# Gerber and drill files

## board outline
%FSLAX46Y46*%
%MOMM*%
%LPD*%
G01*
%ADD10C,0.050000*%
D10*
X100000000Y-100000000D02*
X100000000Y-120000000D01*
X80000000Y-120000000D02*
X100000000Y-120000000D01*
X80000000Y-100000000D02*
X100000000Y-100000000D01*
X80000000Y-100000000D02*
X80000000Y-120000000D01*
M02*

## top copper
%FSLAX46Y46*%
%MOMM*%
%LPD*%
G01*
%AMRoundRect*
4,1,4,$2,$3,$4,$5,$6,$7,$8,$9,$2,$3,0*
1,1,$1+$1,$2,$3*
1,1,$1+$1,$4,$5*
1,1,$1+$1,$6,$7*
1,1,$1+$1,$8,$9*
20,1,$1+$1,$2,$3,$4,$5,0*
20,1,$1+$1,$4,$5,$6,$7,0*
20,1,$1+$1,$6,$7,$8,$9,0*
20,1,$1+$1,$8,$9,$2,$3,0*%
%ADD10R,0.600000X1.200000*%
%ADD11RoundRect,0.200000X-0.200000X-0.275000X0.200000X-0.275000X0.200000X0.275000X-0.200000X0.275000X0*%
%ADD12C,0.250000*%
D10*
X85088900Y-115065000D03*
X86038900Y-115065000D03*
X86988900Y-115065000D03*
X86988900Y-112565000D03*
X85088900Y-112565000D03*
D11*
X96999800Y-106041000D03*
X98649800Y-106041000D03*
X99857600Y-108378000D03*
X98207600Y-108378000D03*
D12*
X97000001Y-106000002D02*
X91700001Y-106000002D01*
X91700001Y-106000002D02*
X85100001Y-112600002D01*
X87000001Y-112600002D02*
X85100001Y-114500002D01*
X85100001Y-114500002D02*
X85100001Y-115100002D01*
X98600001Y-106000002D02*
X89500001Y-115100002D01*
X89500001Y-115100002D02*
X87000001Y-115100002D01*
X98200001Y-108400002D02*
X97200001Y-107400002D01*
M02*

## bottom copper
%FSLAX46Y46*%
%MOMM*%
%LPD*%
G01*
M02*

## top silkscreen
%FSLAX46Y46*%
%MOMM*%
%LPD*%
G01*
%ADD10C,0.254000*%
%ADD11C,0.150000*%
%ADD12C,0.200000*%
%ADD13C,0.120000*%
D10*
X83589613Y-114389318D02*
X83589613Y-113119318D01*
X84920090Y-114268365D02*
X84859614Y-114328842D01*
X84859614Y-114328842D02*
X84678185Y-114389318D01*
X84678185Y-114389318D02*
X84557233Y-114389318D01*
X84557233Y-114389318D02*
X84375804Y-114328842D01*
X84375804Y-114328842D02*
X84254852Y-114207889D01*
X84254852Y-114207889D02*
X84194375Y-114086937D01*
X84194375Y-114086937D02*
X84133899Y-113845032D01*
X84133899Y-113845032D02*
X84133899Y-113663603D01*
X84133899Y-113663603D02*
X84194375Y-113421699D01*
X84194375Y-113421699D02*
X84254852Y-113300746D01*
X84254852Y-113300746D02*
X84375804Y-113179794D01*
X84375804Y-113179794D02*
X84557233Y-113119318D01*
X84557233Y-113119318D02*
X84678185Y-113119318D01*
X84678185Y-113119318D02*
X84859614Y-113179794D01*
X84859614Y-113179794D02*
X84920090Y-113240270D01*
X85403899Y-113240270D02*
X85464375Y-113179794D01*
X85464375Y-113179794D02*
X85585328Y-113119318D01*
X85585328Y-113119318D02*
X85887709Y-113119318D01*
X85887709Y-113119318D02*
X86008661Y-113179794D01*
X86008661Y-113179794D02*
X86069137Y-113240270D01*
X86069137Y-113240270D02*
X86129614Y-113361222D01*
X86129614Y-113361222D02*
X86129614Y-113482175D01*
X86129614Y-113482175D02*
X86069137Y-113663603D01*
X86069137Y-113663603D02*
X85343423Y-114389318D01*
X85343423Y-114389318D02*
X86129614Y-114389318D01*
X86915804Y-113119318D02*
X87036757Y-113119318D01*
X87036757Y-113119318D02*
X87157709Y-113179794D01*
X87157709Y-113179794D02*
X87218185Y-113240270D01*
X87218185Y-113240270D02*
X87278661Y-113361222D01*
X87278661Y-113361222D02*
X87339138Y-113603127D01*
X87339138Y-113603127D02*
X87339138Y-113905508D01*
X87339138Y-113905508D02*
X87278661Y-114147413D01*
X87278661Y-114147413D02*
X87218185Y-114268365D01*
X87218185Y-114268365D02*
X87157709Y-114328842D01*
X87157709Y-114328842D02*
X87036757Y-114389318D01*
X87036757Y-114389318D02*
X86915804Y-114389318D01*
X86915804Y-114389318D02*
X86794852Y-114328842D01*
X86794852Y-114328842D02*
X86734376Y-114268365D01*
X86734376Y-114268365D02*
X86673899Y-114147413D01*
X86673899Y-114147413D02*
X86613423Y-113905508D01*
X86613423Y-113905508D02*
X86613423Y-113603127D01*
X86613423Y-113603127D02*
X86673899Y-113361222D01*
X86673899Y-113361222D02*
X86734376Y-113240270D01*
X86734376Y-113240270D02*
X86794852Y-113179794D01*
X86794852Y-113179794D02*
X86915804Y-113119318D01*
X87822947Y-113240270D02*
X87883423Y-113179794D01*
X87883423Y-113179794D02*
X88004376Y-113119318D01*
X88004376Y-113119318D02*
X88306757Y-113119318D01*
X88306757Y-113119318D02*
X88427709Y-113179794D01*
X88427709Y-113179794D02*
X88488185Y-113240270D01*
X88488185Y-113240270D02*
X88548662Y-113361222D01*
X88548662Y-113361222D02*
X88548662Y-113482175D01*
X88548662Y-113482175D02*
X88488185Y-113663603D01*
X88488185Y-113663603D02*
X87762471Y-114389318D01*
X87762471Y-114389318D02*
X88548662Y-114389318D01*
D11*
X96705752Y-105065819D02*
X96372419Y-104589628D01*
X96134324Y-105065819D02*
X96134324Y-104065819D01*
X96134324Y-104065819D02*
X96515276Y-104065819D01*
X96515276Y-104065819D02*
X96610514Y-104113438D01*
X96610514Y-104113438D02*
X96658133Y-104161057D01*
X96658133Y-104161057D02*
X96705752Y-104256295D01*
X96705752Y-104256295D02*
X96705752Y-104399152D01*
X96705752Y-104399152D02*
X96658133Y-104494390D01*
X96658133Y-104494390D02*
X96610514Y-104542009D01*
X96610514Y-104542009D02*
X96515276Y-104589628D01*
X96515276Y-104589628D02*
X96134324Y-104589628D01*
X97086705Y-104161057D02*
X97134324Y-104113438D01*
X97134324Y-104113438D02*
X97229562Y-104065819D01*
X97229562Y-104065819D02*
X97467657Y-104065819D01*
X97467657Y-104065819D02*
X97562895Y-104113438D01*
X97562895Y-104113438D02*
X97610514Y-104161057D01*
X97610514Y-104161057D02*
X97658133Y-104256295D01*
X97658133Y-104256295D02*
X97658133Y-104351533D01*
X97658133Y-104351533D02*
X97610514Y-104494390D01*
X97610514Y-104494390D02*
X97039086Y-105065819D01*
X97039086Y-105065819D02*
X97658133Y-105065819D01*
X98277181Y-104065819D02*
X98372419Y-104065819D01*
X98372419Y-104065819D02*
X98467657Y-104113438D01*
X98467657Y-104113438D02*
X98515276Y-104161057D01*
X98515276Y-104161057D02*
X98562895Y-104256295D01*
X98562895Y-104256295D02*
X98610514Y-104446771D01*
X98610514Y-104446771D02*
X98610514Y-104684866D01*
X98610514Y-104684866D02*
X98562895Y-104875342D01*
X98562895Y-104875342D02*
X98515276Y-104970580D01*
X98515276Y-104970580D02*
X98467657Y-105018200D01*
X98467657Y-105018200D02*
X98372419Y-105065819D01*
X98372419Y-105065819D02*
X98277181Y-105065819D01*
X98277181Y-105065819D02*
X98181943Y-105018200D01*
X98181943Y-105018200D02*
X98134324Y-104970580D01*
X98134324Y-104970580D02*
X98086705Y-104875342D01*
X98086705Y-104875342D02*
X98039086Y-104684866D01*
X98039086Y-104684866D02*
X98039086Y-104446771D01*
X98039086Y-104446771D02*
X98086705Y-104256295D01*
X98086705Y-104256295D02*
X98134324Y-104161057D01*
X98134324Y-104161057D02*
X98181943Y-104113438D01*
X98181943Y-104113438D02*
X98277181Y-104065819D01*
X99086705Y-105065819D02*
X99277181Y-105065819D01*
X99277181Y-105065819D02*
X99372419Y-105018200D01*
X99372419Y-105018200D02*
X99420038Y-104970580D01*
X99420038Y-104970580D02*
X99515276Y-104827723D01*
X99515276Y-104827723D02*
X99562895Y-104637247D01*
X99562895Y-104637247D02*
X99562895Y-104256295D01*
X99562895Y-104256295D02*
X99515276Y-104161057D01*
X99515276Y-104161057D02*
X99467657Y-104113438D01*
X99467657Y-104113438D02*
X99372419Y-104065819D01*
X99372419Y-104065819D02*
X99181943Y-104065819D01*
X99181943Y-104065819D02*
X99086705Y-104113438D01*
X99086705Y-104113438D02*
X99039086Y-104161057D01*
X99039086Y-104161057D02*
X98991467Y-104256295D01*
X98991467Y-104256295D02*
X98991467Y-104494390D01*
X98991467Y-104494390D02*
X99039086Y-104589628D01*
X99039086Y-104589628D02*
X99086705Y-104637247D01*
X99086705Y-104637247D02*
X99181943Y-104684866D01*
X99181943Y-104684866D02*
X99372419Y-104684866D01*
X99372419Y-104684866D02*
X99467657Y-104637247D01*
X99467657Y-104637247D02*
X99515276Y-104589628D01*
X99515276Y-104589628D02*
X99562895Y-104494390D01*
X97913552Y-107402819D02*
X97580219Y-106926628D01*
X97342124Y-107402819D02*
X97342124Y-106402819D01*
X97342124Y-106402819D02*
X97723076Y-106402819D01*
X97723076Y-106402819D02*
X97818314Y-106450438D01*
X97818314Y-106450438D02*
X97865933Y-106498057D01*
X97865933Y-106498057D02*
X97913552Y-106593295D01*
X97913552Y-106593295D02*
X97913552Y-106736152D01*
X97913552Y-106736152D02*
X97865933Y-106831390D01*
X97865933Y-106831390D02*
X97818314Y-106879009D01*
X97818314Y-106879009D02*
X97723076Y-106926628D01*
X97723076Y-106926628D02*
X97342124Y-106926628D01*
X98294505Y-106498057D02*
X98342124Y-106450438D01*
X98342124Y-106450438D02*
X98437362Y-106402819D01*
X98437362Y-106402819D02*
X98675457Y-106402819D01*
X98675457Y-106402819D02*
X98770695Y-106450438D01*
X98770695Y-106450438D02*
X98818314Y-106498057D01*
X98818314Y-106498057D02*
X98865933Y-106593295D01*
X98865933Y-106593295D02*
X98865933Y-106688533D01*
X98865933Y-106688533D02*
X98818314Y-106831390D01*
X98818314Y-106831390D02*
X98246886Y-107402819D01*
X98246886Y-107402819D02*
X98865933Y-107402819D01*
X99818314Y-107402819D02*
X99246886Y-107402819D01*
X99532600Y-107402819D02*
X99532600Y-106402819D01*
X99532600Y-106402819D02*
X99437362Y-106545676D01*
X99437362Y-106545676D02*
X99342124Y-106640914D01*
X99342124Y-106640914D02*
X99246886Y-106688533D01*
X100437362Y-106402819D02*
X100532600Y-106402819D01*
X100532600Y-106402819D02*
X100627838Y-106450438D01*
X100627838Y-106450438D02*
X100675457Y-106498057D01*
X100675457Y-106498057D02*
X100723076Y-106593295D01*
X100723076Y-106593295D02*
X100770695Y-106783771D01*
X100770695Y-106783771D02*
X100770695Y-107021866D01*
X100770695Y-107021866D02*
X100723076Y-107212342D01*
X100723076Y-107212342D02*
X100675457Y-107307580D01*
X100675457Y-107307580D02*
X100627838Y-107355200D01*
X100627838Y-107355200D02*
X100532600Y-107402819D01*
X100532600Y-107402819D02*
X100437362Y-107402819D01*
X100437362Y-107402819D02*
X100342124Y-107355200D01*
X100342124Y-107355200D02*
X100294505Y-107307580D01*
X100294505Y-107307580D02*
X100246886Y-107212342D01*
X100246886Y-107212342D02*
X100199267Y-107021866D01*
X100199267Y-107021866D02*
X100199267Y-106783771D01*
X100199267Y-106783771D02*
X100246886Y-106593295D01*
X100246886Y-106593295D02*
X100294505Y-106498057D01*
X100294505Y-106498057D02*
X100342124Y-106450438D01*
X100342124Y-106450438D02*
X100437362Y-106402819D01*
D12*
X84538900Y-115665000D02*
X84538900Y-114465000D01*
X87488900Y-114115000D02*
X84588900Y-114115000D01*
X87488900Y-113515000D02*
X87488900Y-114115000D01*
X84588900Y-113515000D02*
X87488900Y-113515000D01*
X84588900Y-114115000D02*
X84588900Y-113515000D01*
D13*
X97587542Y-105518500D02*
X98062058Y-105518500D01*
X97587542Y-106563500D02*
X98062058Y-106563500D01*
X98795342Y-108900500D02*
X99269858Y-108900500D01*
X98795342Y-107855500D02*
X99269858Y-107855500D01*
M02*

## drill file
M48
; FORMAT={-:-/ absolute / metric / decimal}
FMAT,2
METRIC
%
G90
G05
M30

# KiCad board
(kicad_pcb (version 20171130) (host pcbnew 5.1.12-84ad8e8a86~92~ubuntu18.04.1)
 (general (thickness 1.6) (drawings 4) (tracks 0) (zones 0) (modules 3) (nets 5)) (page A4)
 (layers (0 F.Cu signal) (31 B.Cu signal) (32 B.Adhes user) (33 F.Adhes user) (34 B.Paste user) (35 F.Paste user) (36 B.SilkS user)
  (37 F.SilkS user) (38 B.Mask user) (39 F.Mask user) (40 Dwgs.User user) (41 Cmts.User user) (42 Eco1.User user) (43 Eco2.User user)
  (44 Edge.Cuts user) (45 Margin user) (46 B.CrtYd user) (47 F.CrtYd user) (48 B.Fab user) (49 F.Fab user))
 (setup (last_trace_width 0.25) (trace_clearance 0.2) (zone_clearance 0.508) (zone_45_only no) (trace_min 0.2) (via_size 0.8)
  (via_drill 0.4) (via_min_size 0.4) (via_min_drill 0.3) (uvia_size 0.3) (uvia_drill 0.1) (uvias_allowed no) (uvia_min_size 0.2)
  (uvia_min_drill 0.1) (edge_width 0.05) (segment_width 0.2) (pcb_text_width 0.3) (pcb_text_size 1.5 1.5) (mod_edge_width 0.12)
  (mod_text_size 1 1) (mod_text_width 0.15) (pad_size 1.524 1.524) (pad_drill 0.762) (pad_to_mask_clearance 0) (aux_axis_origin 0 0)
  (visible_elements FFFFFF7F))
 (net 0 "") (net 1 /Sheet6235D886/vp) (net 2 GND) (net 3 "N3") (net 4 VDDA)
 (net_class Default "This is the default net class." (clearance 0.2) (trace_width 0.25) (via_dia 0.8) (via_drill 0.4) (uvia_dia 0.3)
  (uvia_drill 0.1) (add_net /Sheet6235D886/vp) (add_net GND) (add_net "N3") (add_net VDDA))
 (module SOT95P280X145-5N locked (layer F.Cu) (at 86.038900 113.815000 90.000000)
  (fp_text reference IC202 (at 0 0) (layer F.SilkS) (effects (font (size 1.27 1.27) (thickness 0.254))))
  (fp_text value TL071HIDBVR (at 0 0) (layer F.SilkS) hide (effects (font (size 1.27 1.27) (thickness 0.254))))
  (fp_line (start -1.85 -1.5) (end -0.65 -1.5) (layer F.SilkS) (width 0.2))
  (fp_line (start -0.3 1.45) (end -0.3 -1.45) (layer F.SilkS) (width 0.2))
  (fp_line (start 0.3 1.45) (end -0.3 1.45) (layer F.SilkS) (width 0.2))
  (fp_line (start 0.3 -1.45) (end 0.3 1.45) (layer F.SilkS) (width 0.2))
  (fp_line (start -0.3 -1.45) (end 0.3 -1.45) (layer F.SilkS) (width 0.2))
  (pad 1 smd rect (at -1.25 -0.95 180.000000) (size 0.6 1.2) (layers F.Cu F.Mask F.Paste) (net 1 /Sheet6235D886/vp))
  (pad 2 smd rect (at -1.25 0 180.000000) (size 0.6 1.2) (layers F.Cu F.Mask F.Paste) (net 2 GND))
  (pad 3 smd rect (at -1.25 0.95 180.000000) (size 0.6 1.2) (layers F.Cu F.Mask F.Paste) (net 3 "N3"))
  (pad 4 smd rect (at 1.25 0.95 180.000000) (size 0.6 1.2) (layers F.Cu F.Mask F.Paste) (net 1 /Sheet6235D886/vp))
  (pad 5 smd rect (at 1.25 -0.95 180.000000) (size 0.6 1.2) (layers F.Cu F.Mask F.Paste) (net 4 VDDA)))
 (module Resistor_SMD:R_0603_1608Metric (layer F.Cu) (at 97.824800 106.041000)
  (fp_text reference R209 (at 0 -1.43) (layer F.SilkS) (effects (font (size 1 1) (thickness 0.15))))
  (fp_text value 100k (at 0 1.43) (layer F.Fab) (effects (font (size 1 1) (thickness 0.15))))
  (fp_line (start -0.237258 -0.5225) (end 0.237258 -0.5225) (layer F.SilkS) (width 0.12))
  (fp_line (start -0.237258 0.5225) (end 0.237258 0.5225) (layer F.SilkS) (width 0.12))
  (pad 1 smd roundrect (at -0.825 0) (size 0.8 0.95) (layers F.Cu F.Mask F.Paste) (roundrect_rratio 0.25) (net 4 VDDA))
  (pad 2 smd roundrect (at 0.825 0) (size 0.8 0.95) (layers F.Cu F.Mask F.Paste) (roundrect_rratio 0.25) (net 3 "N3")))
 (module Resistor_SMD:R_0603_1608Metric (layer F.Cu) (at 99.032600 108.378000)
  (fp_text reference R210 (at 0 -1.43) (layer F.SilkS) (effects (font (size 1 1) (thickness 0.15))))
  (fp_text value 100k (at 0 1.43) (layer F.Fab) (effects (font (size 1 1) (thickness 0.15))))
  (fp_line (start -0.237258 0.5225) (end 0.237258 0.5225) (layer F.SilkS) (width 0.12))
  (fp_line (start -0.237258 -0.5225) (end 0.237258 -0.5225) (layer F.SilkS) (width 0.12))
  (pad 2 smd roundrect (at 0.825 0) (size 0.8 0.95) (layers F.Cu F.Mask F.Paste) (roundrect_rratio 0.25) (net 2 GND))
  (pad 1 smd roundrect (at -0.825 0) (size 0.8 0.95) (layers F.Cu F.Mask F.Paste) (roundrect_rratio 0.25) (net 3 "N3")))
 (gr_line (start 100 100) (end 100 120) (layer Edge.Cuts) (width 0.05))
 (gr_line (start 80 120) (end 100 120) (layer Edge.Cuts) (width 0.05))
 (gr_line (start 80 100) (end 100 100) (layer Edge.Cuts) (width 0.05))
 (gr_line (start 80 100) (end 80 120) (layer Edge.Cuts) (width 0.05))
 (segment (start 97.000001 106.000002) (end 91.700001 106.000002) (width 0.250000) (layer F.Cu) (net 4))
 (segment (start 91.700001 106.000002) (end 85.100001 112.600002) (width 0.250000) (layer F.Cu) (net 4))
 (segment (start 87.000001 112.600002) (end 85.100001 114.500002) (width 0.250000) (layer F.Cu) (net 1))
 (segment (start 85.100001 114.500002) (end 85.100001 115.100002) (width 0.250000) (layer F.Cu) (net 1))
 (segment (start 98.600001 106.000002) (end 89.500001 115.100002) (width 0.250000) (layer F.Cu) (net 3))
 (segment (start 89.500001 115.100002) (end 87.000001 115.100002) (width 0.250000) (layer F.Cu) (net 3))
 (segment (start 98.200001 108.400002) (end 97.200001 107.400002) (width 0.250000) (layer F.Cu) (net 3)))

